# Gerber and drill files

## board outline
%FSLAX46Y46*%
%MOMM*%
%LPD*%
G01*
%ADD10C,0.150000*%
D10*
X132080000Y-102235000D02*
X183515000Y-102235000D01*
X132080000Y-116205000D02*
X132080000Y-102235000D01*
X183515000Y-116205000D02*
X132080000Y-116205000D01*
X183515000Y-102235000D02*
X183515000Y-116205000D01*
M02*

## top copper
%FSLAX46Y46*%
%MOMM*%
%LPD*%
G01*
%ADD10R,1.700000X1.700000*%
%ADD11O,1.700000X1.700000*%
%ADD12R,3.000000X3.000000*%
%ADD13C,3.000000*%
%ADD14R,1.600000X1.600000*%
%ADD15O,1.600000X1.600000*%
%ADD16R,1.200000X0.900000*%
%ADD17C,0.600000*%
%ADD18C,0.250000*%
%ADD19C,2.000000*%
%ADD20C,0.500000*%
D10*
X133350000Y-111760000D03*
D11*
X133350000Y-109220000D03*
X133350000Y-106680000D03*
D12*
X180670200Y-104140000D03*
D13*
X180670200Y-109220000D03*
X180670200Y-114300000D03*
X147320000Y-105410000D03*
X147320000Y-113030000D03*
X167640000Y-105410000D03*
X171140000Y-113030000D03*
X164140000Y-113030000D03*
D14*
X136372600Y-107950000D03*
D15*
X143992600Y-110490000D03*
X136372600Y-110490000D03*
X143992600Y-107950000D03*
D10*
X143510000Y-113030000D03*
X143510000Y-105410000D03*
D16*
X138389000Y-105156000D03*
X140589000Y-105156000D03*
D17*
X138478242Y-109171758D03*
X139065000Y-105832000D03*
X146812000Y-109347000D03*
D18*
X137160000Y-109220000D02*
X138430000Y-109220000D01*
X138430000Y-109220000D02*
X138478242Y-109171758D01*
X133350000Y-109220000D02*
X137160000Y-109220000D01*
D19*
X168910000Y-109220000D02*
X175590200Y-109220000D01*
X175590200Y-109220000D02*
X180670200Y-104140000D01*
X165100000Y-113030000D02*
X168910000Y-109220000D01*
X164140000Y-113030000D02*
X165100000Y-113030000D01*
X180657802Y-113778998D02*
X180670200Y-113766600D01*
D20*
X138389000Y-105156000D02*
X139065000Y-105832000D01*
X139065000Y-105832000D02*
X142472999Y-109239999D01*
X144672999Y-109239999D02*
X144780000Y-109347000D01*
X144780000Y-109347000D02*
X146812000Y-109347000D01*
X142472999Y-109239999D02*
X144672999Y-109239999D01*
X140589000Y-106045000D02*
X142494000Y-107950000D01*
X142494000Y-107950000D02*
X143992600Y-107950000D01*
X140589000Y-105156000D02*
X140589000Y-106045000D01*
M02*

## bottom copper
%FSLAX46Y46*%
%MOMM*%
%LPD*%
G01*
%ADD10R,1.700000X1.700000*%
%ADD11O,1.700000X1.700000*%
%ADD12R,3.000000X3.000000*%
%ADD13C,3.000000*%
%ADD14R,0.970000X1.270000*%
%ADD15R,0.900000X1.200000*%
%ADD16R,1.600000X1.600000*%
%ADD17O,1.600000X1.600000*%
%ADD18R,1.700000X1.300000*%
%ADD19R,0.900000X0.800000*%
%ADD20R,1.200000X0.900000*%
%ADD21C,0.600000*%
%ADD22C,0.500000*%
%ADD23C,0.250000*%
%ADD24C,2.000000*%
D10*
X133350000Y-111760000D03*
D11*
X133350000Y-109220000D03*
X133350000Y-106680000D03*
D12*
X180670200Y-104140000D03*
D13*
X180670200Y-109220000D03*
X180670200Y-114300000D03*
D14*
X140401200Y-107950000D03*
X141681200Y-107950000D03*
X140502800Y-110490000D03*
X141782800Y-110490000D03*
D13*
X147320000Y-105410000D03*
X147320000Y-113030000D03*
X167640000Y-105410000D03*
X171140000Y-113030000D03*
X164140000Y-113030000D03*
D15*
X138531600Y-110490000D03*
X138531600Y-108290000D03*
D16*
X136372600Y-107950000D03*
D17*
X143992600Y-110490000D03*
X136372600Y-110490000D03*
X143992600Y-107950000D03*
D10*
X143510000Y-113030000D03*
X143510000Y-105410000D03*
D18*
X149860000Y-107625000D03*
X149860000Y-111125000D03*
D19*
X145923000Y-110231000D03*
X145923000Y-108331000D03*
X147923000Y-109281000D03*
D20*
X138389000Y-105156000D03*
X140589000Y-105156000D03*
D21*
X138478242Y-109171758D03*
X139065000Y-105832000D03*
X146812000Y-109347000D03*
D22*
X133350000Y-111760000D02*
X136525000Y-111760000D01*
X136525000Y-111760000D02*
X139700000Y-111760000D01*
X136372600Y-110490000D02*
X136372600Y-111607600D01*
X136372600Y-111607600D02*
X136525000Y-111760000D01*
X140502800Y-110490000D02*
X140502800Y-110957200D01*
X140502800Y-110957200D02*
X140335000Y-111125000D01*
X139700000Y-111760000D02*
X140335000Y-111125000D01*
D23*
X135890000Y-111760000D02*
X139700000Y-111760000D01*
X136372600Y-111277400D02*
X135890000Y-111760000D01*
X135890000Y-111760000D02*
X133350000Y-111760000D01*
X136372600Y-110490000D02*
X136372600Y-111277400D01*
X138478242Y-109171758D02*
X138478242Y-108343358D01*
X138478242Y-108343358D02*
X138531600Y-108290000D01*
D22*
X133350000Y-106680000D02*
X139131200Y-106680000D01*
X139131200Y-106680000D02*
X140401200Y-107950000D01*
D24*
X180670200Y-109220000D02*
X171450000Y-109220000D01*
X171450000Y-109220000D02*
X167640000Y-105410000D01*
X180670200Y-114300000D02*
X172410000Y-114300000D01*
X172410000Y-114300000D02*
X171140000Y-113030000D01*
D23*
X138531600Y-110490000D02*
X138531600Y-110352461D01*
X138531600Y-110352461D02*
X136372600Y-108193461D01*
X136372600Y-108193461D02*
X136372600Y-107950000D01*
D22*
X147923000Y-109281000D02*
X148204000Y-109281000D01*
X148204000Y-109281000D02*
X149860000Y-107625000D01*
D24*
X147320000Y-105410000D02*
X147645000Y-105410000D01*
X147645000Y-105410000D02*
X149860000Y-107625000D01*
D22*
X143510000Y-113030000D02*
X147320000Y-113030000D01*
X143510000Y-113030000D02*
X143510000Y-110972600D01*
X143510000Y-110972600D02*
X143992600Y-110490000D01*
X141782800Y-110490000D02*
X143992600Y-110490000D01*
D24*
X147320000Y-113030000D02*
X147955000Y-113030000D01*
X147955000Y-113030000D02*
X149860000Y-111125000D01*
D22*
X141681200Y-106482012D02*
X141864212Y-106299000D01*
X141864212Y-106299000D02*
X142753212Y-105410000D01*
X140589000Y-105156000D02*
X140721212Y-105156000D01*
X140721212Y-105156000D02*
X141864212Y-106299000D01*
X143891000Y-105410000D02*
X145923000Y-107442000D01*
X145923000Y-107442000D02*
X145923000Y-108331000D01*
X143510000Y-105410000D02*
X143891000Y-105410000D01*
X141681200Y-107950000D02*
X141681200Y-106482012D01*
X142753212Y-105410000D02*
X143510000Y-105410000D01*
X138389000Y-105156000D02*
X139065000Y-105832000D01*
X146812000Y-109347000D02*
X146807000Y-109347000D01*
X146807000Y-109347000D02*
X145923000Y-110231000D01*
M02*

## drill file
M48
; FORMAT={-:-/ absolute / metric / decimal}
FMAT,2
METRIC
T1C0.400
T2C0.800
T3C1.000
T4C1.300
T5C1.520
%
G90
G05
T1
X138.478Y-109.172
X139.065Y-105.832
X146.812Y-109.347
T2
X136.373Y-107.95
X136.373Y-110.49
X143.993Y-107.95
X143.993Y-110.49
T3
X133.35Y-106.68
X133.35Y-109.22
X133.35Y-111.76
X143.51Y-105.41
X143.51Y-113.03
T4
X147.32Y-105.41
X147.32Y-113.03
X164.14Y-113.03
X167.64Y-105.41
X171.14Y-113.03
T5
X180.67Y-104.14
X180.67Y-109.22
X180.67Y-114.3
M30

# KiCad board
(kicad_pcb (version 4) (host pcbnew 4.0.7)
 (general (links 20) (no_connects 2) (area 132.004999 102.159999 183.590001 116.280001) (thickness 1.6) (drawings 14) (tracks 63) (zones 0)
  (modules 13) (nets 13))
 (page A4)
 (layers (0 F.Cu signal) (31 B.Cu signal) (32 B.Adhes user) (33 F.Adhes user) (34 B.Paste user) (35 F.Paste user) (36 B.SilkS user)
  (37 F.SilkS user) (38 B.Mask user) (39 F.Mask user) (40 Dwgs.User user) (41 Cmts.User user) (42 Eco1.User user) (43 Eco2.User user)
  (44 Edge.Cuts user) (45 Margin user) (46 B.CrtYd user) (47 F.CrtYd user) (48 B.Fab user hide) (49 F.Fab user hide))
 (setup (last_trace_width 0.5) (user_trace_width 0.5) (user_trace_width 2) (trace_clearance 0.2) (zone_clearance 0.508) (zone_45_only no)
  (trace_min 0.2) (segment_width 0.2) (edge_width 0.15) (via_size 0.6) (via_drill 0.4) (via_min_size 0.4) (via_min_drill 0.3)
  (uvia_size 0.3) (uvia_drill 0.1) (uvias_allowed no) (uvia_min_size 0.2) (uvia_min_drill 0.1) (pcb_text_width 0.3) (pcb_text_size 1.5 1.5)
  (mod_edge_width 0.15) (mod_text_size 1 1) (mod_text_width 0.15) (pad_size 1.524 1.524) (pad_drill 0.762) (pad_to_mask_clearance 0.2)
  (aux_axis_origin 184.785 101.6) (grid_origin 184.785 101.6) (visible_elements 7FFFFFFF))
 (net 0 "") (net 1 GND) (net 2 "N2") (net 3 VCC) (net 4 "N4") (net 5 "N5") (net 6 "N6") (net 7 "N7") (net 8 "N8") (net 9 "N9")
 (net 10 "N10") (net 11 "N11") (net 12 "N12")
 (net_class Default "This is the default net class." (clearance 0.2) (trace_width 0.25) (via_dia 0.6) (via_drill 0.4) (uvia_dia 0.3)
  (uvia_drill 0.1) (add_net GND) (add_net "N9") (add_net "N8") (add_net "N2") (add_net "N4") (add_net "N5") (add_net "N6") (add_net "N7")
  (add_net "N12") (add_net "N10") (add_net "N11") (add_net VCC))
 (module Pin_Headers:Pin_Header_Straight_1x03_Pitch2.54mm (layer F.Cu) (at 133.35 111.76 180)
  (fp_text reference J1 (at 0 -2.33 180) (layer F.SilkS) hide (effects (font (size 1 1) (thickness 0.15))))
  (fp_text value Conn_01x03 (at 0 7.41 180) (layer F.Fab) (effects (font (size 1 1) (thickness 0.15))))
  (pad 1 thru_hole rect (at 0 0 180) (size 1.7 1.7) (drill 1) (layers *.Cu *.Mask) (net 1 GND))
  (pad 2 thru_hole oval (at 0 2.54 180) (size 1.7 1.7) (drill 1) (layers *.Cu *.Mask) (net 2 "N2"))
  (pad 3 thru_hole oval (at 0 5.08 180) (size 1.7 1.7) (drill 1) (layers *.Cu *.Mask) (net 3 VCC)))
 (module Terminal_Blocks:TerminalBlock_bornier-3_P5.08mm (layer F.Cu) (at 180.6702 104.14 270)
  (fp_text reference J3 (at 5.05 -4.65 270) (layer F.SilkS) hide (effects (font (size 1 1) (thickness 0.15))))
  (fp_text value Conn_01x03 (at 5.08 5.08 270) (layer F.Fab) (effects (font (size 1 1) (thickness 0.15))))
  (pad 1 thru_hole rect (at 0 0 270) (size 3 3) (drill 1.52) (layers *.Cu *.Mask) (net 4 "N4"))
  (pad 2 thru_hole circle (at 5.08 0 270) (size 3 3) (drill 1.52) (layers *.Cu *.Mask) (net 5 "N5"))
  (pad 3 thru_hole circle (at 10.16 0 270) (size 3 3) (drill 1.52) (layers *.Cu *.Mask) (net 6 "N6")))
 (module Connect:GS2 (layer B.Cu) (at 141.0412 107.95 270)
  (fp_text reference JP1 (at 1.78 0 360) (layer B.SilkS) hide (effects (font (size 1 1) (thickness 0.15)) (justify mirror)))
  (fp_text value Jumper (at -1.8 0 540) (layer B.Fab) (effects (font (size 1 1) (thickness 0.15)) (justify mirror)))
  (pad 1 smd rect (at 0 0.64 270) (size 1.27 0.97) (layers B.Cu B.Paste B.Mask) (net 3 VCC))
  (pad 2 smd rect (at 0 -0.64 270) (size 1.27 0.97) (layers B.Cu B.Paste B.Mask) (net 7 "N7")))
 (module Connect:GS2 (layer B.Cu) (at 141.1428 110.49 270)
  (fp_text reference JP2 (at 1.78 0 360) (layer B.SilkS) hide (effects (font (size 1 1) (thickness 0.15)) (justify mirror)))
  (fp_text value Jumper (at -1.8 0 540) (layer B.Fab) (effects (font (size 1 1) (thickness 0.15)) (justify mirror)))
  (pad 1 smd rect (at 0 0.64 270) (size 1.27 0.97) (layers B.Cu B.Paste B.Mask) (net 1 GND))
  (pad 2 smd rect (at 0 -0.64 270) (size 1.27 0.97) (layers B.Cu B.Paste B.Mask) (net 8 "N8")))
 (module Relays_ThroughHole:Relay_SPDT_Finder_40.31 (layer F.Cu) (at 147.32 105.41)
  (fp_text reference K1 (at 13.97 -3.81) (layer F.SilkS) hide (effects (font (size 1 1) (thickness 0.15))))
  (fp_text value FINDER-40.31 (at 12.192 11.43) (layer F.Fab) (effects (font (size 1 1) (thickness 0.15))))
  (pad A1 thru_hole circle (at 0 0) (size 3 3) (drill 1.3) (layers *.Cu *.Mask) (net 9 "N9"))
  (pad A2 thru_hole circle (at 0 7.62) (size 3 3) (drill 1.3) (layers *.Cu *.Mask) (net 8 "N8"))
  (pad 11 thru_hole circle (at 20.32 0) (size 3 3) (drill 1.3) (layers *.Cu *.Mask) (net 5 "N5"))
  (pad 14 thru_hole circle (at 23.82 7.62) (size 3 3) (drill 1.3) (layers *.Cu *.Mask) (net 6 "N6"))
  (pad 12 thru_hole circle (at 16.82 7.62) (size 3 3) (drill 1.3) (layers *.Cu *.Mask) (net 4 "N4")))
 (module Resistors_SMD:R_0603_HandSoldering (layer B.Cu) (at 138.5316 109.39 90)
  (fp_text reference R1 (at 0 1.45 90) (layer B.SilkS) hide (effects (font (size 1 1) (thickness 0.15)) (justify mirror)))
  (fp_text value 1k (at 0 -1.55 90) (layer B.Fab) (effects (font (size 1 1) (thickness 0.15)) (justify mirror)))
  (pad 1 smd rect (at -1.1 0 90) (size 1.2 0.9) (layers B.Cu B.Paste B.Mask) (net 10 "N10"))
  (pad 2 smd rect (at 1.1 0 90) (size 1.2 0.9) (layers B.Cu B.Paste B.Mask) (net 2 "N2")))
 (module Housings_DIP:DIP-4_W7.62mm (layer F.Cu) (at 136.3726 107.95)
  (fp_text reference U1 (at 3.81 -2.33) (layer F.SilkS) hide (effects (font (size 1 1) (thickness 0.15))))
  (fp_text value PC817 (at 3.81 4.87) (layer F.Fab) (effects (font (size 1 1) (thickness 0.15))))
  (pad 1 thru_hole rect (at 0 0) (size 1.6 1.6) (drill 0.8) (layers *.Cu *.Mask) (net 10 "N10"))
  (pad 3 thru_hole oval (at 7.62 2.54) (size 1.6 1.6) (drill 0.8) (layers *.Cu *.Mask) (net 8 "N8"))
  (pad 2 thru_hole oval (at 0 2.54) (size 1.6 1.6) (drill 0.8) (layers *.Cu *.Mask) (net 1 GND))
  (pad 4 thru_hole oval (at 7.62 0) (size 1.6 1.6) (drill 0.8) (layers *.Cu *.Mask) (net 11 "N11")))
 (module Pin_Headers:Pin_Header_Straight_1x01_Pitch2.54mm (layer F.Cu) (at 143.51 113.03 90)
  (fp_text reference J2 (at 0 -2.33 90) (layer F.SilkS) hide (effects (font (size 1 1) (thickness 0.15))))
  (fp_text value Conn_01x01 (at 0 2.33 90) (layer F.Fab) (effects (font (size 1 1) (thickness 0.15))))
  (pad 1 thru_hole rect (at 0 0 90) (size 1.7 1.7) (drill 1) (layers *.Cu *.Mask) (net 8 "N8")))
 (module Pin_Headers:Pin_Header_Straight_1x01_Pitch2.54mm (layer F.Cu) (at 143.51 105.41)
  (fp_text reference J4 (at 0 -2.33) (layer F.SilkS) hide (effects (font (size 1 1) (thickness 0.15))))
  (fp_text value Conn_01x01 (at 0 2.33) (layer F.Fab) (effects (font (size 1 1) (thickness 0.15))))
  (pad 1 thru_hole rect (at 0 0) (size 1.7 1.7) (drill 1) (layers *.Cu *.Mask) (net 7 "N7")))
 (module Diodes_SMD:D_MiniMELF (layer B.Cu) (at 149.86 109.375 270)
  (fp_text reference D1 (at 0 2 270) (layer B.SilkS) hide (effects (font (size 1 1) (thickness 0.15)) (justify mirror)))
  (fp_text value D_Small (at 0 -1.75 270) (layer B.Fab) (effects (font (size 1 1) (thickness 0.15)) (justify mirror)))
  (pad 1 smd rect (at -1.75 0 270) (size 1.3 1.7) (layers B.Cu B.Paste B.Mask) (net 9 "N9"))
  (pad 2 smd rect (at 1.75 0 270) (size 1.3 1.7) (layers B.Cu B.Paste B.Mask) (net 8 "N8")))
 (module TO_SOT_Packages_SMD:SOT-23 (layer B.Cu) (at 146.923 109.281)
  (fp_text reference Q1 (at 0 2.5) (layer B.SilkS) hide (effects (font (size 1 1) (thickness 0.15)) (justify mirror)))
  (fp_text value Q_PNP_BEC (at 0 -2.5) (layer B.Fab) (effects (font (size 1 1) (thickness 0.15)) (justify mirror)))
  (pad 1 smd rect (at -1 0.95) (size 0.9 0.8) (layers B.Cu B.Paste B.Mask) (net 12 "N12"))
  (pad 2 smd rect (at -1 -0.95) (size 0.9 0.8) (layers B.Cu B.Paste B.Mask) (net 7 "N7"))
  (pad 3 smd rect (at 1 0) (size 0.9 0.8) (layers B.Cu B.Paste B.Mask) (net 9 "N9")))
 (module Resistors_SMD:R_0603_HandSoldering (layer F.Cu) (at 139.489 105.156)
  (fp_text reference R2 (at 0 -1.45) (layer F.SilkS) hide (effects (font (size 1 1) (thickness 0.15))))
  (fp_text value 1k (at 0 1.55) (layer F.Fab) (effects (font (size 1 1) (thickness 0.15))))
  (pad 1 smd rect (at -1.1 0) (size 1.2 0.9) (layers F.Cu F.Paste F.Mask) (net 12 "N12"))
  (pad 2 smd rect (at 1.1 0) (size 1.2 0.9) (layers F.Cu F.Paste F.Mask) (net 11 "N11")))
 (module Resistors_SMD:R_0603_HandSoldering (layer B.Cu) (at 139.489 105.156)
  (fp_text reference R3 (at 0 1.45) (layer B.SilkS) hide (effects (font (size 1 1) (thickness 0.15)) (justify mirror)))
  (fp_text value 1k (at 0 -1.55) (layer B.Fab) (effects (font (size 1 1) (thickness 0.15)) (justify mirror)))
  (pad 1 smd rect (at -1.1 0) (size 1.2 0.9) (layers B.Cu B.Paste B.Mask) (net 12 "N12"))
  (pad 2 smd rect (at 1.1 0) (size 1.2 0.9) (layers B.Cu B.Paste B.Mask) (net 7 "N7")))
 (gr_line (start 132.08 102.235) (end 183.515 102.235) (layer Edge.Cuts) (width 0.15))
 (gr_line (start 132.08 116.205) (end 132.08 102.235) (layer Edge.Cuts) (width 0.15))
 (gr_line (start 183.515 116.205) (end 132.08 116.205) (layer Edge.Cuts) (width 0.15))
 (gr_line (start 183.515 102.235) (end 183.515 116.205) (layer Edge.Cuts) (width 0.15))
 (segment (start 133.35 111.76) (end 136.525 111.76) (width 0.5) (layer B.Cu) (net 1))
 (segment (start 136.525 111.76) (end 139.7 111.76) (width 0.5) (layer B.Cu) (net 1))
 (segment (start 136.3726 110.49) (end 136.3726 111.6076) (width 0.5) (layer B.Cu) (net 1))
 (segment (start 136.3726 111.6076) (end 136.525 111.76) (width 0.5) (layer B.Cu) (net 1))
 (segment (start 140.5028 110.49) (end 140.5028 110.9572) (width 0.5) (layer B.Cu) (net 1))
 (segment (start 140.5028 110.9572) (end 140.335 111.125) (width 0.5) (layer B.Cu) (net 1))
 (segment (start 139.7 111.76) (end 140.335 111.125) (width 0.5) (layer B.Cu) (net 1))
 (segment (start 135.89 111.76) (end 139.7 111.76) (width 0.25) (layer B.Cu) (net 1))
 (segment (start 136.3726 111.2774) (end 135.89 111.76) (width 0.25) (layer B.Cu) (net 1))
 (segment (start 135.89 111.76) (end 133.35 111.76) (width 0.25) (layer B.Cu) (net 1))
 (segment (start 136.3726 110.49) (end 136.3726 111.2774) (width 0.25) (layer B.Cu) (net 1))
 (segment (start 138.478242 109.171758) (end 138.478242 108.343358) (width 0.25) (layer B.Cu) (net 2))
 (segment (start 138.478242 108.343358) (end 138.5316 108.29) (width 0.25) (layer B.Cu) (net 2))
 (segment (start 137.16 109.22) (end 138.43 109.22) (width 0.25) (layer F.Cu) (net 2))
 (segment (start 138.43 109.22) (end 138.478242 109.171758) (width 0.25) (layer F.Cu) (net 2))
 (via (at 138.478242 109.171758) (size 0.6) (drill 0.4) (layers F.Cu B.Cu) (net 2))
 (segment (start 133.35 109.22) (end 137.16 109.22) (width 0.25) (layer F.Cu) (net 2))
 (segment (start 133.35 106.68) (end 139.1312 106.68) (width 0.5) (layer B.Cu) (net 3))
 (segment (start 139.1312 106.68) (end 140.4012 107.95) (width 0.5) (layer B.Cu) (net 3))
 (segment (start 168.91 109.22) (end 175.5902 109.22) (width 2) (layer F.Cu) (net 4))
 (segment (start 175.5902 109.22) (end 180.6702 104.14) (width 2) (layer F.Cu) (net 4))
 (segment (start 165.1 113.03) (end 168.91 109.22) (width 2) (layer F.Cu) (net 4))
 (segment (start 164.14 113.03) (end 165.1 113.03) (width 2) (layer F.Cu) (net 4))
 (segment (start 180.6702 109.22) (end 171.45 109.22) (width 2) (layer B.Cu) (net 5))
 (segment (start 171.45 109.22) (end 167.64 105.41) (width 2) (layer B.Cu) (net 5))
 (segment (start 180.6702 114.3) (end 172.41 114.3) (width 2) (layer B.Cu) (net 6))
 (segment (start 172.41 114.3) (end 171.14 113.03) (width 2) (layer B.Cu) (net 6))
 (segment (start 180.657802 113.778998) (end 180.6702 113.7666) (width 2) (layer F.Cu) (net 6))
 (segment (start 138.5316 110.49) (end 138.5316 110.352461) (width 0.25) (layer B.Cu) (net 10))
 (segment (start 138.5316 110.352461) (end 136.3726 108.193461) (width 0.25) (layer B.Cu) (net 10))
 (segment (start 136.3726 108.193461) (end 136.3726 107.95) (width 0.25) (layer B.Cu) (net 10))
 (segment (start 147.923 109.281) (end 148.204 109.281) (width 0.5) (layer B.Cu) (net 9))
 (segment (start 148.204 109.281) (end 149.86 107.625) (width 0.5) (layer B.Cu) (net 9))
 (segment (start 147.32 105.41) (end 147.645 105.41) (width 2) (layer B.Cu) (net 9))
 (segment (start 147.645 105.41) (end 149.86 107.625) (width 2) (layer B.Cu) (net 9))
 (segment (start 143.51 113.03) (end 147.32 113.03) (width 0.5) (layer B.Cu) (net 8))
 (segment (start 143.51 113.03) (end 143.51 110.9726) (width 0.5) (layer B.Cu) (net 8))
 (segment (start 143.51 110.9726) (end 143.9926 110.49) (width 0.5) (layer B.Cu) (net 8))
 (segment (start 141.7828 110.49) (end 143.9926 110.49) (width 0.5) (layer B.Cu) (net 8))
 (segment (start 147.32 113.03) (end 147.955 113.03) (width 2) (layer B.Cu) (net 8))
 (segment (start 147.955 113.03) (end 149.86 111.125) (width 2) (layer B.Cu) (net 8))
 (segment (start 141.6812 106.482012) (end 141.864212 106.299) (width 0.5) (layer B.Cu) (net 7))
 (segment (start 141.864212 106.299) (end 142.753212 105.41) (width 0.5) (layer B.Cu) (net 7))
 (segment (start 140.589 105.156) (end 140.721212 105.156) (width 0.5) (layer B.Cu) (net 7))
 (segment (start 140.721212 105.156) (end 141.864212 106.299) (width 0.5) (layer B.Cu) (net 7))
 (segment (start 143.891 105.41) (end 145.923 107.442) (width 0.5) (layer B.Cu) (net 7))
 (segment (start 145.923 107.442) (end 145.923 108.331) (width 0.5) (layer B.Cu) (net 7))
 (segment (start 143.51 105.41) (end 143.891 105.41) (width 0.5) (layer B.Cu) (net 7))
 (segment (start 141.6812 107.95) (end 141.6812 106.482012) (width 0.5) (layer B.Cu) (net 7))
 (segment (start 142.753212 105.41) (end 143.51 105.41) (width 0.5) (layer B.Cu) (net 7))
 (segment (start 138.389 105.156) (end 139.065 105.832) (width 0.5) (layer F.Cu) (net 12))
 (segment (start 139.065 105.832) (end 142.472999 109.239999) (width 0.5) (layer F.Cu) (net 12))
 (segment (start 138.389 105.156) (end 139.065 105.832) (width 0.5) (layer B.Cu) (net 12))
 (via (at 139.065 105.832) (size 0.6) (drill 0.4) (layers F.Cu B.Cu) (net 12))
 (segment (start 146.812 109.347) (end 146.807 109.347) (width 0.5) (layer B.Cu) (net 12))
 (segment (start 146.807 109.347) (end 145.923 110.231) (width 0.5) (layer B.Cu) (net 12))
 (segment (start 144.672999 109.239999) (end 144.78 109.347) (width 0.5) (layer F.Cu) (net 12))
 (segment (start 144.78 109.347) (end 146.812 109.347) (width 0.5) (layer F.Cu) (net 12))
 (via (at 146.812 109.347) (size 0.6) (drill 0.4) (layers F.Cu B.Cu) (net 12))
 (segment (start 142.472999 109.239999) (end 144.672999 109.239999) (width 0.5) (layer F.Cu) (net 12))
 (segment (start 140.589 106.045) (end 142.494 107.95) (width 0.5) (layer F.Cu) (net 11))
 (segment (start 142.494 107.95) (end 143.9926 107.95) (width 0.5) (layer F.Cu) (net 11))
 (segment (start 140.589 105.156) (end 140.589 106.045) (width 0.5) (layer F.Cu) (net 11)))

